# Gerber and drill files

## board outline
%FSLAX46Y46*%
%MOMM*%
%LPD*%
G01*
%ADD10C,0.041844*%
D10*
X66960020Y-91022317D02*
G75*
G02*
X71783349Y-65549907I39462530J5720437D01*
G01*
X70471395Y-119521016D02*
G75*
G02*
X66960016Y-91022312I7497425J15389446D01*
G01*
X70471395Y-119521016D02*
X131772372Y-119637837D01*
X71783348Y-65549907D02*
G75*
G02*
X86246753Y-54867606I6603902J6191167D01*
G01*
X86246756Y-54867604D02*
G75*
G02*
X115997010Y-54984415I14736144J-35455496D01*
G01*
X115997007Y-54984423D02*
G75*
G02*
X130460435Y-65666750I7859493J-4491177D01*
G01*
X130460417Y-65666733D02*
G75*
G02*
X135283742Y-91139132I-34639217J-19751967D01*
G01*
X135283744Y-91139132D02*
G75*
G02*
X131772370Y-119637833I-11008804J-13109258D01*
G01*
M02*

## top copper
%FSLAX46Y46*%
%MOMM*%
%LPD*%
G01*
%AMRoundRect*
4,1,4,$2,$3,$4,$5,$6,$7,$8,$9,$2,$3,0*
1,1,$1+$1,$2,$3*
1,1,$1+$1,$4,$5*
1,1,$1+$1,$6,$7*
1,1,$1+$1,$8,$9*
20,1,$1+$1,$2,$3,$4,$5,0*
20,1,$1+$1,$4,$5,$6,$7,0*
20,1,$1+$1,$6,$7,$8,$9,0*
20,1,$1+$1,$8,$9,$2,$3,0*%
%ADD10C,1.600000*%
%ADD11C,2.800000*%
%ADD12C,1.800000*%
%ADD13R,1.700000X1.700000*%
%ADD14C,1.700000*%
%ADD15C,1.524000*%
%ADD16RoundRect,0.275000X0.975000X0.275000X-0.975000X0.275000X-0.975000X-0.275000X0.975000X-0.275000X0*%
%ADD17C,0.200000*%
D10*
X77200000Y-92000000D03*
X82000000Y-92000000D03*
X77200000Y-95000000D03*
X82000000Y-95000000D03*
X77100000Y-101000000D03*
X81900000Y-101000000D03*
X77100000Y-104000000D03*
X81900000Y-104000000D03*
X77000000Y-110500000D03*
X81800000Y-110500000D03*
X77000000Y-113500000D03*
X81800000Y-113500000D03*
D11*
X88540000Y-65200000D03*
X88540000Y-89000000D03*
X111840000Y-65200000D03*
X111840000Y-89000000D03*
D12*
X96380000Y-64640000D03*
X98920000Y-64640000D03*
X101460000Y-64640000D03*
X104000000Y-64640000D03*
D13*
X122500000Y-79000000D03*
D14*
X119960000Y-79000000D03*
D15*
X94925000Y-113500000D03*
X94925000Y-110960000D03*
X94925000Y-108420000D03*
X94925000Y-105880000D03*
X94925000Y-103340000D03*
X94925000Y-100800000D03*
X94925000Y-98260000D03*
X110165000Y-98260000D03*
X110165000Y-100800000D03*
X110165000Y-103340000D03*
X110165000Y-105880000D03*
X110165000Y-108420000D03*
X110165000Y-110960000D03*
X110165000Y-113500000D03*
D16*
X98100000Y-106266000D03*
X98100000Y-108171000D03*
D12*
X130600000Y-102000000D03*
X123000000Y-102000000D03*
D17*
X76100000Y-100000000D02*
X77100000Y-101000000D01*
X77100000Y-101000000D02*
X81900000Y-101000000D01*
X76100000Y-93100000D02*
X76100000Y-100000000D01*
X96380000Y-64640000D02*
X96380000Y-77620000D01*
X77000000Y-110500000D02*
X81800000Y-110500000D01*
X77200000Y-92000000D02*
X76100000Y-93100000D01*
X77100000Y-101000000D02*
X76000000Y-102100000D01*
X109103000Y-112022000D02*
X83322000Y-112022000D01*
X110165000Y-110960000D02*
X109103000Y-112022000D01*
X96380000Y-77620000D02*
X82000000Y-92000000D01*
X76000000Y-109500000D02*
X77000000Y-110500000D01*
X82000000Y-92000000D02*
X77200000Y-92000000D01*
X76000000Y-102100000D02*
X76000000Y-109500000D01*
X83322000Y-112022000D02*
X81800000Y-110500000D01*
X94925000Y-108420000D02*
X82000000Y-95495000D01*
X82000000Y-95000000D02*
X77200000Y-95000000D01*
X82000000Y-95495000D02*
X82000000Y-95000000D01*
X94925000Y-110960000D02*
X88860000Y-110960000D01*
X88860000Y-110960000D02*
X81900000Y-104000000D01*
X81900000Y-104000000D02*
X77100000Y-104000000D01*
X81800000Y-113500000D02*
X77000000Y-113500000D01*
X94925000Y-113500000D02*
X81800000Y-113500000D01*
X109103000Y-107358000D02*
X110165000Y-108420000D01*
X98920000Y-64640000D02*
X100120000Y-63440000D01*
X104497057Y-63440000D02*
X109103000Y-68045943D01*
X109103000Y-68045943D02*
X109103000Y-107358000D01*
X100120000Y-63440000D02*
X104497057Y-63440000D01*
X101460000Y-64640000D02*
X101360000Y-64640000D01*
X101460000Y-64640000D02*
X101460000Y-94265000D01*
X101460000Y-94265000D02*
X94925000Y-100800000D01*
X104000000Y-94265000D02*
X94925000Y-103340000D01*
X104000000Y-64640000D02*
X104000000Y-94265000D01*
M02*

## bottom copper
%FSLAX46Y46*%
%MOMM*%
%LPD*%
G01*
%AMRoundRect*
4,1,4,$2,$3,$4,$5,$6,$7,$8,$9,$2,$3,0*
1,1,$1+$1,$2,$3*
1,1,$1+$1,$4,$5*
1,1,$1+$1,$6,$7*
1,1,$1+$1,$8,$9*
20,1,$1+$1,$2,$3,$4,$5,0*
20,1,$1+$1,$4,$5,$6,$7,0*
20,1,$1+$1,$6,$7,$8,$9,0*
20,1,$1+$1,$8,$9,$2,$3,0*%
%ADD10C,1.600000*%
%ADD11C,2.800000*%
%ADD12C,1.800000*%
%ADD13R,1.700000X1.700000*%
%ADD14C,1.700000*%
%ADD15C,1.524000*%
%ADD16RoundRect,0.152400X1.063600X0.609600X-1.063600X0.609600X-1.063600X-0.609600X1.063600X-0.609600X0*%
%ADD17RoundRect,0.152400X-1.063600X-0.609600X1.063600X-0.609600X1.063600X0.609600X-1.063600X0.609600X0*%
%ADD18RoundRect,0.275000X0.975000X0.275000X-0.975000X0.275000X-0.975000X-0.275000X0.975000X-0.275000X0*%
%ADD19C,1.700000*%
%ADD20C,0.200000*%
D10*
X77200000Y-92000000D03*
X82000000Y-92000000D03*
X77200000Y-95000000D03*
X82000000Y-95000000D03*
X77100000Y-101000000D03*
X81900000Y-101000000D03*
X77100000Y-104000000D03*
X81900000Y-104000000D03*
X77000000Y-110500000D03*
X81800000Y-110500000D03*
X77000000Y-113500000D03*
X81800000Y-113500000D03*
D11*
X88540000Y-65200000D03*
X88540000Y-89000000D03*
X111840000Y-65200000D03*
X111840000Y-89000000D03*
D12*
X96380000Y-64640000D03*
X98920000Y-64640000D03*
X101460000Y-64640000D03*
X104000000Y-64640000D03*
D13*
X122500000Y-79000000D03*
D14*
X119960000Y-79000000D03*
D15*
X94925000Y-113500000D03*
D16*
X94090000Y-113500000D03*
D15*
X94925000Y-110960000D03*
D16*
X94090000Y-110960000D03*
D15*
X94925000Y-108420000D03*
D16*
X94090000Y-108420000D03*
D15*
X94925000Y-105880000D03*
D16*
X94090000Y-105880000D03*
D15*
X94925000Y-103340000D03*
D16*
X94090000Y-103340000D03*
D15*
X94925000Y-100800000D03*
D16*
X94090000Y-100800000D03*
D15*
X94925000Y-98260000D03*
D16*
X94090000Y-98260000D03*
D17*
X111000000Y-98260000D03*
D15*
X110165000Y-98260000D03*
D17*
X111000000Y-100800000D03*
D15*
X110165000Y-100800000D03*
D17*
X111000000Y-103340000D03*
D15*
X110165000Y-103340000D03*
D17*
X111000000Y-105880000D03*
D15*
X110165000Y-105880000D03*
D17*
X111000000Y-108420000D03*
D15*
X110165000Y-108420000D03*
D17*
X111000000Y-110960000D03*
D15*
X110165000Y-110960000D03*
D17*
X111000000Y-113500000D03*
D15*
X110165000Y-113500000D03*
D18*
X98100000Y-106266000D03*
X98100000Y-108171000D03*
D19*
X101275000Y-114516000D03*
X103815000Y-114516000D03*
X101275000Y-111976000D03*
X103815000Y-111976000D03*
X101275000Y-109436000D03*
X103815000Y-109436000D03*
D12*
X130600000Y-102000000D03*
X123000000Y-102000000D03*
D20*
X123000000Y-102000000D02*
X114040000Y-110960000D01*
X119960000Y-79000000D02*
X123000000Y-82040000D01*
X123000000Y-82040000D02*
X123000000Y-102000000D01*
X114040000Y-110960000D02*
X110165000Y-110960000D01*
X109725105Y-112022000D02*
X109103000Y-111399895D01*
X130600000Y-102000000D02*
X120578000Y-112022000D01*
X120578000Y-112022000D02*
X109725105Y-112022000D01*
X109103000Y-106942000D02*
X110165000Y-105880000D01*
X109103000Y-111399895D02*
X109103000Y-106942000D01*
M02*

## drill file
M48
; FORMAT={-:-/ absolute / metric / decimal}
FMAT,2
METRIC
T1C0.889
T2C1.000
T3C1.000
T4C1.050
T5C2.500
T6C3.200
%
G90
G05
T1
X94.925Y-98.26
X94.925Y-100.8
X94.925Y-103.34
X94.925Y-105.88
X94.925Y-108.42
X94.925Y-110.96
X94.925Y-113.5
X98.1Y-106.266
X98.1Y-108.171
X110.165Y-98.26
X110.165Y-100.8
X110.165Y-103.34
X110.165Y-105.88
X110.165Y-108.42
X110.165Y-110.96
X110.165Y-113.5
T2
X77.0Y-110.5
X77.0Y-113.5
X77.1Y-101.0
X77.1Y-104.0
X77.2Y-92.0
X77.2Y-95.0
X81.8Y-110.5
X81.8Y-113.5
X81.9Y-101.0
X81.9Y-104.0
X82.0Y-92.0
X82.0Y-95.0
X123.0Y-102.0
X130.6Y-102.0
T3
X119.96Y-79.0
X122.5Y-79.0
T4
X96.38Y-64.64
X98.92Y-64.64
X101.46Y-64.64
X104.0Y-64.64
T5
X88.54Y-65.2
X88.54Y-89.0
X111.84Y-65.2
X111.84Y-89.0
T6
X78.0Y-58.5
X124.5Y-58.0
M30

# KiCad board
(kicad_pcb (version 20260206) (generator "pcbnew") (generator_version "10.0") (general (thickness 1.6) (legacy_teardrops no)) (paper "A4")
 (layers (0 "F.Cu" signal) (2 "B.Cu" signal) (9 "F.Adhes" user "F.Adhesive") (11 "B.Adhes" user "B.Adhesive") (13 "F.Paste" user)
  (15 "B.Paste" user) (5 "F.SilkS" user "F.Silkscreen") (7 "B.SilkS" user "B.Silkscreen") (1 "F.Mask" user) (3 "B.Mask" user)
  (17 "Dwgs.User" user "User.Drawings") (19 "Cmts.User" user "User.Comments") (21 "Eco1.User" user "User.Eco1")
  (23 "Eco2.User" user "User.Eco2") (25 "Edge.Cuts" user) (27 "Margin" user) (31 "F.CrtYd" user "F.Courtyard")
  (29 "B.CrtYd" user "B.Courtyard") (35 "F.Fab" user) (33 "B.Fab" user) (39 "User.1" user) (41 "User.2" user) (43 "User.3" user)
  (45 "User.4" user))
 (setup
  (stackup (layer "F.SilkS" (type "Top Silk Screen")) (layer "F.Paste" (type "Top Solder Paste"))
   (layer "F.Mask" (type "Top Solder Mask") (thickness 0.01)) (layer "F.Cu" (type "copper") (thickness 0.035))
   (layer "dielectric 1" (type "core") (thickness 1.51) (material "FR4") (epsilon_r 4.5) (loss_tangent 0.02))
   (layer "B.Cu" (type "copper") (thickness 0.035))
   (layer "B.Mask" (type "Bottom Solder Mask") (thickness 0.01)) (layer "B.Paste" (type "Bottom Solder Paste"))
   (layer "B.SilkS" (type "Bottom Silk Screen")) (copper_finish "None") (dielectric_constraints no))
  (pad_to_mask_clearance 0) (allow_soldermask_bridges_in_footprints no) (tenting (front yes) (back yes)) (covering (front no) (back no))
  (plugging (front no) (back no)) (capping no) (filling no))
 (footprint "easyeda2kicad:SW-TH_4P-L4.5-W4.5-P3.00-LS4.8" (layer "F.Cu") (at 79.6 93.5)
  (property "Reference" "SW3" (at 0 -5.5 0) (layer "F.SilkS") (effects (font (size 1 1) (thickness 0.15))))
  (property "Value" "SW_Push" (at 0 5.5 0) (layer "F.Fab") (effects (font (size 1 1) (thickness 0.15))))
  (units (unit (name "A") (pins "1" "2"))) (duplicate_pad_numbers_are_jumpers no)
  (pad "1" thru_hole circle (at -2.4 -1.5) (size 1.6 1.6) (drill 0.999998) (layers "*.Cu" "*.Mask") (remove_unused_layers no) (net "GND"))
  (pad "1" thru_hole circle (at 2.4 -1.5) (size 1.6 1.6) (drill 0.999998) (layers "*.Cu" "*.Mask") (remove_unused_layers no) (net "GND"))
  (pad "2" thru_hole circle (at -2.4 1.5) (size 1.6 1.6) (drill 0.999998) (layers "*.Cu" "*.Mask") (remove_unused_layers no)
   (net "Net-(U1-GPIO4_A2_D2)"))
  (pad "2" thru_hole circle (at 2.4 1.5) (size 1.6 1.6) (drill 0.999998) (layers "*.Cu" "*.Mask") (remove_unused_layers no)
   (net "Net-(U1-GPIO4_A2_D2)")))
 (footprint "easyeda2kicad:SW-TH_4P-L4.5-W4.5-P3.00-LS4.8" (layer "F.Cu") (at 79.5 102.5)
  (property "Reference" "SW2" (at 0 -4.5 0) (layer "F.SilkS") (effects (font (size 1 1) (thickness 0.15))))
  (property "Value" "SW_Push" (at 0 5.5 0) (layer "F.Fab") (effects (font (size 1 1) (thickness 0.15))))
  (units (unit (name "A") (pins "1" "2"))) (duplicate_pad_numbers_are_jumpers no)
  (pad "1" thru_hole circle (at -2.4 -1.5) (size 1.6 1.6) (drill 0.999998) (layers "*.Cu" "*.Mask") (remove_unused_layers no) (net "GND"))
  (pad "1" thru_hole circle (at 2.4 -1.5) (size 1.6 1.6) (drill 0.999998) (layers "*.Cu" "*.Mask") (remove_unused_layers no) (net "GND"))
  (pad "2" thru_hole circle (at -2.4 1.5) (size 1.6 1.6) (drill 0.999998) (layers "*.Cu" "*.Mask") (remove_unused_layers no)
   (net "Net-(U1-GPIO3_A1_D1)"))
  (pad "2" thru_hole circle (at 2.4 1.5) (size 1.6 1.6) (drill 0.999998) (layers "*.Cu" "*.Mask") (remove_unused_layers no)
   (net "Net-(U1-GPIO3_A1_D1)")))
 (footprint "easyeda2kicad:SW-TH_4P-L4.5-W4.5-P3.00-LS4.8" (layer "F.Cu") (at 79.4 112)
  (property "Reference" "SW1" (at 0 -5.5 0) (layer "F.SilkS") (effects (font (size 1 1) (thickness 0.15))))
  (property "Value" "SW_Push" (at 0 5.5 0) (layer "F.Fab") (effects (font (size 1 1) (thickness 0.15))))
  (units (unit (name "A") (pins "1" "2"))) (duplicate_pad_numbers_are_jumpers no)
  (pad "1" thru_hole circle (at -2.4 -1.5) (size 1.6 1.6) (drill 0.999998) (layers "*.Cu" "*.Mask") (remove_unused_layers no) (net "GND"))
  (pad "1" thru_hole circle (at 2.4 -1.5) (size 1.6 1.6) (drill 0.999998) (layers "*.Cu" "*.Mask") (remove_unused_layers no) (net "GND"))
  (pad "2" thru_hole circle (at -2.4 1.5) (size 1.6 1.6) (drill 0.999998) (layers "*.Cu" "*.Mask") (remove_unused_layers no)
   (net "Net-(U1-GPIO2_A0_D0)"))
  (pad "2" thru_hole circle (at 2.4 1.5) (size 1.6 1.6) (drill 0.999998) (layers "*.Cu" "*.Mask") (remove_unused_layers no)
   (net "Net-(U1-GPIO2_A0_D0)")))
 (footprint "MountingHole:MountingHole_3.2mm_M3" (layer "F.Cu") (at 78 58.5)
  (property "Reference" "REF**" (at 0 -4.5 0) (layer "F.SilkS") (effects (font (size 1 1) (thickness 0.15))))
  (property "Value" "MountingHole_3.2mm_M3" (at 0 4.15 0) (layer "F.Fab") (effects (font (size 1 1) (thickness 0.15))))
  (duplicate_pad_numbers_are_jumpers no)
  (pad "" np_thru_hole circle (at 0 0) (size 3.2 3.2) (drill 3.2) (layers "*.Cu" "*.Mask")))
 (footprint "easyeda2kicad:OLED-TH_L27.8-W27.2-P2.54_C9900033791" (layer "F.Cu") (at 100.19 64.64)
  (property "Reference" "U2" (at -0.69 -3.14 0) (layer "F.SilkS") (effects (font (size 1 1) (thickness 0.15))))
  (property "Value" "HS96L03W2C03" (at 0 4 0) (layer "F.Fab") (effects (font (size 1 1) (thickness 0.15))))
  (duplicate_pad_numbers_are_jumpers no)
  (pad "" thru_hole circle (at -11.65 0.56) (size 2.8 2.8) (drill 2.5) (layers "*.Cu" "*.Mask") (remove_unused_layers no))
  (pad "" thru_hole circle (at -11.65 24.36) (size 2.8 2.8) (drill 2.5) (layers "*.Cu" "*.Mask") (remove_unused_layers no))
  (pad "" thru_hole circle (at 11.65 0.56) (size 2.8 2.8) (drill 2.5) (layers "*.Cu" "*.Mask") (remove_unused_layers no))
  (pad "" thru_hole circle (at 11.65 24.36) (size 2.8 2.8) (drill 2.5) (layers "*.Cu" "*.Mask") (remove_unused_layers no))
  (pad "1" thru_hole circle (at -3.81 0) (size 1.8 1.8) (drill 1.049986) (layers "*.Cu" "*.Mask") (remove_unused_layers no) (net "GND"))
  (pad "2" thru_hole circle (at -1.27 0) (size 1.8 1.8) (drill 1.049986) (layers "*.Cu" "*.Mask") (remove_unused_layers no) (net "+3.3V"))
  (pad "3" thru_hole circle (at 1.27 0) (size 1.8 1.8) (drill 1.049986) (layers "*.Cu" "*.Mask") (remove_unused_layers no)
   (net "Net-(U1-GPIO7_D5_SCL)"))
  (pad "4" thru_hole circle (at 3.81 0) (size 1.8 1.8) (drill 1.049986) (layers "*.Cu" "*.Mask") (remove_unused_layers no)
   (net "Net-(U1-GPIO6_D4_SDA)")))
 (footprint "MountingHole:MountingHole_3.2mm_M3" (layer "F.Cu") (at 124.5 58)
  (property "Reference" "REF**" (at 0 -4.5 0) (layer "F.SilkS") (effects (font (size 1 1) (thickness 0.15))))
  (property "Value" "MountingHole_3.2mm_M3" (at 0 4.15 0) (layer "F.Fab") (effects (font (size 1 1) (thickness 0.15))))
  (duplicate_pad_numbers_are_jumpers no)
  (pad "" np_thru_hole circle (at 0 0) (size 3.2 3.2) (drill 3.2) (layers "*.Cu" "*.Mask")))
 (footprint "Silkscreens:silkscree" (layer "F.Cu") (at 76 75)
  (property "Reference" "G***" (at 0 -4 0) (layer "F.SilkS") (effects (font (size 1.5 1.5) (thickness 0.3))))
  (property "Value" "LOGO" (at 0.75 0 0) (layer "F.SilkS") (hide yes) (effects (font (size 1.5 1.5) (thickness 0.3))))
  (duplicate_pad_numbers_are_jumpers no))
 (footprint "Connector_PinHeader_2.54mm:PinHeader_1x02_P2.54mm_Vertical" (layer "B.Cu") (at 122.5 79 90)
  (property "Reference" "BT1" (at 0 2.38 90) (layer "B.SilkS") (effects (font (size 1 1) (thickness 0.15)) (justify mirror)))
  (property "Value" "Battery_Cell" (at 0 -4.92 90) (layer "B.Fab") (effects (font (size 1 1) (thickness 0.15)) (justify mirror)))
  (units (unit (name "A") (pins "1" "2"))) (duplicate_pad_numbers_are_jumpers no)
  (pad "1" thru_hole rect (at 0 0 90) (size 1.7 1.7) (drill 1) (layers "*.Cu" "*.Mask") (remove_unused_layers no) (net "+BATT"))
  (pad "2" thru_hole circle (at 0 -2.54 90) (size 1.7 1.7) (drill 1) (layers "*.Cu" "*.Mask") (remove_unused_layers no) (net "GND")))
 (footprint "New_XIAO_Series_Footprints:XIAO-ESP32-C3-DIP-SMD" (layer "B.Cu") (at 102.545 105.88 -90)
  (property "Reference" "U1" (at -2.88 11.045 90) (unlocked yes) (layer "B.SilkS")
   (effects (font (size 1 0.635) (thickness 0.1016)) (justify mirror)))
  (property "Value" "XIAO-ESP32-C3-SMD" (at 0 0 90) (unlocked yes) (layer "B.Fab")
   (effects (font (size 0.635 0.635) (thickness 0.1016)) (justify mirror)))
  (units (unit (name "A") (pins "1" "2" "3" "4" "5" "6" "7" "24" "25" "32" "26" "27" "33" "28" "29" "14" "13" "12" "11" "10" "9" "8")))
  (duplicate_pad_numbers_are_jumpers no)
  (pad "1" thru_hole circle (at 7.62 7.62 180) (size 1.524 1.524) (drill 0.889) (layers "*.Cu" "*.Mask") (remove_unused_layers no)
   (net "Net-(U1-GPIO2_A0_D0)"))
  (pad "1" smd roundrect (at 7.62 8.455 180) (size 2.432 1.524) (layers "B.Cu" "B.Mask") (roundrect_rratio 0.1) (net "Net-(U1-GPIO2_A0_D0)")
   (thermal_bridge_angle 45))
  (pad "2" thru_hole circle (at 5.08 7.62 180) (size 1.524 1.524) (drill 0.889) (layers "*.Cu" "*.Mask") (remove_unused_layers no)
   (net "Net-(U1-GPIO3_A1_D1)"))
  (pad "2" smd roundrect (at 5.08 8.455 180) (size 2.432 1.524) (layers "B.Cu" "B.Mask") (roundrect_rratio 0.1) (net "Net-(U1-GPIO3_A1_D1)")
   (thermal_bridge_angle 45))
  (pad "3" thru_hole circle (at 2.54 7.62 180) (size 1.524 1.524) (drill 0.889) (layers "*.Cu" "*.Mask") (remove_unused_layers no)
   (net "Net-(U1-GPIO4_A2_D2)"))
  (pad "3" smd roundrect (at 2.54 8.455 180) (size 2.432 1.524) (layers "B.Cu" "B.Mask") (roundrect_rratio 0.1) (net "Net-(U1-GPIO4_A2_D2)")
   (thermal_bridge_angle 45))
  (pad "4" thru_hole circle (at 0 7.62 180) (size 1.524 1.524) (drill 0.889) (layers "*.Cu" "*.Mask") (remove_unused_layers no)
   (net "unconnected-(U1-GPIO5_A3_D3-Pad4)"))
  (pad "4" smd roundrect (at 0 8.455 180) (size 2.432 1.524) (layers "B.Cu" "B.Mask") (roundrect_rratio 0.1)
   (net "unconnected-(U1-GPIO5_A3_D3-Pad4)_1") (thermal_bridge_angle 45))
  (pad "5" thru_hole circle (at -2.54 7.62 180) (size 1.524 1.524) (drill 0.889) (layers "*.Cu" "*.Mask") (remove_unused_layers no)
   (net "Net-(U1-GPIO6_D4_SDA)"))
  (pad "5" smd roundrect (at -2.54 8.455 180) (size 2.432 1.524) (layers "B.Cu" "B.Mask") (roundrect_rratio 0.1)
   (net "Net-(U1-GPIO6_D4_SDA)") (thermal_bridge_angle 45))
  (pad "6" thru_hole circle (at -5.08 7.62 180) (size 1.524 1.524) (drill 0.889) (layers "*.Cu" "*.Mask") (remove_unused_layers no)
   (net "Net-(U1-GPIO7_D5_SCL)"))
  (pad "6" smd roundrect (at -5.08 8.455 180) (size 2.432 1.524) (layers "B.Cu" "B.Mask") (roundrect_rratio 0.1)
   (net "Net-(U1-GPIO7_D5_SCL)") (thermal_bridge_angle 45))
  (pad "7" thru_hole circle (at -7.62 7.62 180) (size 1.524 1.524) (drill 0.889) (layers "*.Cu" "*.Mask") (remove_unused_layers no)
   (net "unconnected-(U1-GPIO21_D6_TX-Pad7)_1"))
  (pad "7" smd roundrect (at -7.62 8.455 180) (size 2.432 1.524) (layers "B.Cu" "B.Mask") (roundrect_rratio 0.1)
   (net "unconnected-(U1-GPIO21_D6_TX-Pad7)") (thermal_bridge_angle 45))
  (pad "8" smd roundrect (at -7.62 -8.455) (size 2.432 1.524) (layers "B.Cu" "B.Mask") (roundrect_rratio 0.1)
   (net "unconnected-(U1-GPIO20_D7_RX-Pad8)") (thermal_bridge_angle 45))
  (pad "8" thru_hole circle (at -7.62 -7.62) (size 1.524 1.524) (drill 0.889) (layers "*.Cu" "*.Mask") (remove_unused_layers no)
   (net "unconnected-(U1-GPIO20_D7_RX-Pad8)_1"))
  (pad "9" smd roundrect (at -5.08 -8.455) (size 2.432 1.524) (layers "B.Cu" "B.Mask") (roundrect_rratio 0.1)
   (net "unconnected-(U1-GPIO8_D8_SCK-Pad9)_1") (thermal_bridge_angle 45))
  (pad "9" thru_hole circle (at -5.08 -7.62) (size 1.524 1.524) (drill 0.889) (layers "*.Cu" "*.Mask") (remove_unused_layers no)
   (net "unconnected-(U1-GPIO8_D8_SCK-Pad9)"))
  (pad "10" smd roundrect (at -2.54 -8.455) (size 2.432 1.524) (layers "B.Cu" "B.Mask") (roundrect_rratio 0.1)
   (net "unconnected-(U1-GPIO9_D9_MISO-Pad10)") (thermal_bridge_angle 45))
  (pad "10" thru_hole circle (at -2.54 -7.62) (size 1.524 1.524) (drill 0.889) (layers "*.Cu" "*.Mask") (remove_unused_layers no)
   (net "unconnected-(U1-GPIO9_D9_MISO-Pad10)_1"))
  (pad "11" smd roundrect (at 0 -8.455) (size 2.432 1.524) (layers "B.Cu" "B.Mask") (roundrect_rratio 0.1) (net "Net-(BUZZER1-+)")
   (thermal_bridge_angle 45))
  (pad "11" thru_hole circle (at 0 -7.62) (size 1.524 1.524) (drill 0.889) (layers "*.Cu" "*.Mask") (remove_unused_layers no)
   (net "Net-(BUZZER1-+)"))
  (pad "12" smd roundrect (at 2.54 -8.455) (size 2.432 1.524) (layers "B.Cu" "B.Mask") (roundrect_rratio 0.1) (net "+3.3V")
   (thermal_bridge_angle 45))
  (pad "12" thru_hole circle (at 2.54 -7.62) (size 1.524 1.524) (drill 0.889) (layers "*.Cu" "*.Mask") (remove_unused_layers no)
   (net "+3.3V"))
  (pad "13" smd roundrect (at 5.08 -8.455) (size 2.432 1.524) (layers "B.Cu" "B.Mask") (roundrect_rratio 0.1) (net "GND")
   (thermal_bridge_angle 45))
  (pad "13" thru_hole circle (at 5.08 -7.62) (size 1.524 1.524) (drill 0.889) (layers "*.Cu" "*.Mask") (remove_unused_layers no) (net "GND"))
  (pad "14" smd roundrect (at 7.62 -8.455) (size 2.432 1.524) (layers "B.Cu" "B.Mask") (roundrect_rratio 0.1) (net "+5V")
   (thermal_bridge_angle 45))
  (pad "14" thru_hole circle (at 7.62 -7.62) (size 1.524 1.524) (drill 0.889) (layers "*.Cu" "*.Mask") (remove_unused_layers no) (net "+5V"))
  (pad "15" thru_hole roundrect (at 0.386 4.445 180) (size 2.5 1.1) (drill 0.889) (layers "*.Cu" "*.Mask") (remove_unused_layers no)
   (roundrect_rratio 0.25) (thermal_bridge_angle 45))
  (pad "16" thru_hole roundrect (at 2.291 4.445 180) (size 2.5 1.1) (drill 0.889) (layers "*.Cu" "*.Mask") (remove_unused_layers no)
   (roundrect_rratio 0.25) (thermal_bridge_angle 45))
  (pad "17" smd circle (at 8.636 1.27) (size 1.7 1.7) (layers "B.Cu" "B.Mask" "B.Paste"))
  (pad "18" smd circle (at 8.636 -1.27) (size 1.7 1.7) (layers "B.Cu" "B.Mask" "B.Paste"))
  (pad "19" smd circle (at 6.096 1.27) (size 1.7 1.7) (layers "B.Cu" "B.Mask" "B.Paste"))
  (pad "20" smd circle (at 6.096 -1.27) (size 1.7 1.7) (layers "B.Cu" "B.Mask" "B.Paste"))
  (pad "21" smd circle (at 3.556 1.27) (size 1.7 1.7) (layers "B.Cu" "B.Mask" "B.Paste"))
  (pad "22" smd circle (at 3.556 -1.27) (size 1.7 1.7) (layers "B.Cu" "B.Mask" "B.Paste")))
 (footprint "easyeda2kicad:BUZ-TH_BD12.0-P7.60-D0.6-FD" (layer "B.Cu") (at 126.8 102 180)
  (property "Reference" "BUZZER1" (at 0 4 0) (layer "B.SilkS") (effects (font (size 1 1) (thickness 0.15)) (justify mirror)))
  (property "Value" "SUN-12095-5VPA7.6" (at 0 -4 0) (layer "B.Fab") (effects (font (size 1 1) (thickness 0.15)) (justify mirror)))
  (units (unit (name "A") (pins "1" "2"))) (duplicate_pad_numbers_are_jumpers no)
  (pad "1" thru_hole circle (at -3.8 0 180) (size 1.8 1.8) (drill 0.999998) (layers "*.Cu" "*.Mask") (remove_unused_layers no)
   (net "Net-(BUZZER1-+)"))
  (pad "2" thru_hole circle (at 3.8 0 180) (size 1.8 1.8) (drill 0.999998) (layers "*.Cu" "*.Mask") (remove_unused_layers no) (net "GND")))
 (gr_arc (start 66.96002 91.022317) (mid 67.24376 77.883179) (end 71.783348 65.549907) (stroke (width 0.041844) (type default))
  (layer "Edge.Cuts"))
 (gr_arc (start 70.471395 119.521016) (mid 60.978702 106.224956) (end 66.96002 91.022317) (stroke (width 0.041844) (type default))
  (layer "Edge.Cuts"))
 (gr_line (start 70.471395 119.521016) (end 131.772372 119.637837) (stroke (width 0.041844) (type default)) (layer "Edge.Cuts"))
 (gr_arc (start 71.783348 65.549907) (mid 73.009334 52.077252) (end 86.246756 54.867604) (stroke (width 0.041844) (type default))
  (layer "Edge.Cuts"))
 (gr_arc (start 86.246756 54.867604) (mid 101.133655 51.92749) (end 115.997007 54.984423) (stroke (width 0.041844) (type default))
  (layer "Edge.Cuts"))
 (gr_arc (start 115.997007 54.984423) (mid 129.234435 52.194078) (end 130.460417 65.666733) (stroke (width 0.041844) (type default))
  (layer "Edge.Cuts"))
 (gr_arc (start 130.460417 65.666733) (mid 135 78) (end 135.283744 91.139132) (stroke (width 0.041844) (type default)) (layer "Edge.Cuts"))
 (gr_arc (start 135.283744 91.139132) (mid 141.265063 106.341772) (end 131.772372 119.637837) (stroke (width 0.041844) (type default))
  (layer "Edge.Cuts"))
 (segment (start 76.1 100) (end 77.1 101) (width 0.2) (layer "F.Cu") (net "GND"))
 (segment (start 77.1 101) (end 81.9 101) (width 0.2) (layer "F.Cu") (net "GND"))
 (segment (start 76.1 93.1) (end 76.1 100) (width 0.2) (layer "F.Cu") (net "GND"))
 (segment (start 96.38 64.64) (end 96.38 77.62) (width 0.2) (layer "F.Cu") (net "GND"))
 (segment (start 77 110.5) (end 81.8 110.5) (width 0.2) (layer "F.Cu") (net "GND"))
 (segment (start 77.2 92) (end 76.1 93.1) (width 0.2) (layer "F.Cu") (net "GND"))
 (segment (start 77.1 101) (end 76 102.1) (width 0.2) (layer "F.Cu") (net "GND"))
 (segment (start 109.103 112.022) (end 83.322 112.022) (width 0.2) (layer "F.Cu") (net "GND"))
 (segment (start 110.165 110.96) (end 109.103 112.022) (width 0.2) (layer "F.Cu") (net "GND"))
 (segment (start 96.38 77.62) (end 82 92) (width 0.2) (layer "F.Cu") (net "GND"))
 (segment (start 76 109.5) (end 77 110.5) (width 0.2) (layer "F.Cu") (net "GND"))
 (segment (start 82 92) (end 77.2 92) (width 0.2) (layer "F.Cu") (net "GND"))
 (segment (start 76 102.1) (end 76 109.5) (width 0.2) (layer "F.Cu") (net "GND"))
 (segment (start 83.322 112.022) (end 81.8 110.5) (width 0.2) (layer "F.Cu") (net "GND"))
 (segment (start 123 102) (end 114.04 110.96) (width 0.2) (layer "B.Cu") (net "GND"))
 (segment (start 119.96 79) (end 123 82.04) (width 0.2) (layer "B.Cu") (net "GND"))
 (segment (start 123 82.04) (end 123 102) (width 0.2) (layer "B.Cu") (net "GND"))
 (segment (start 114.04 110.96) (end 110.165 110.96) (width 0.2) (layer "B.Cu") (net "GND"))
 (segment (start 94.925 108.42) (end 82 95.495) (width 0.2) (layer "F.Cu") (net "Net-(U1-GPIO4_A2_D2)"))
 (segment (start 82 95) (end 77.2 95) (width 0.2) (layer "F.Cu") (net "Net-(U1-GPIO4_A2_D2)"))
 (segment (start 82 95.495) (end 82 95) (width 0.2) (layer "F.Cu") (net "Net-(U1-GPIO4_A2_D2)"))
 (segment (start 109.725105 112.022) (end 109.103 111.399895) (width 0.2) (layer "B.Cu") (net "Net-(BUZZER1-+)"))
 (segment (start 130.6 102) (end 120.578 112.022) (width 0.2) (layer "B.Cu") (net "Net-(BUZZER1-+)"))
 (segment (start 120.578 112.022) (end 109.725105 112.022) (width 0.2) (layer "B.Cu") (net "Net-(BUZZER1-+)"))
 (segment (start 109.103 106.942) (end 110.165 105.88) (width 0.2) (layer "B.Cu") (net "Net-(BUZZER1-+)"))
 (segment (start 109.103 111.399895) (end 109.103 106.942) (width 0.2) (layer "B.Cu") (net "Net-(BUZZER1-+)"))
 (segment (start 94.925 110.96) (end 88.86 110.96) (width 0.2) (layer "F.Cu") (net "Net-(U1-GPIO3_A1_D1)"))
 (segment (start 88.86 110.96) (end 81.9 104) (width 0.2) (layer "F.Cu") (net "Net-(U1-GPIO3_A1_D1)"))
 (segment (start 81.9 104) (end 77.1 104) (width 0.2) (layer "F.Cu") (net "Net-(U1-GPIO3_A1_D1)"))
 (segment (start 81.8 113.5) (end 77 113.5) (width 0.2) (layer "F.Cu") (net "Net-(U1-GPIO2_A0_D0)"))
 (segment (start 94.925 113.5) (end 81.8 113.5) (width 0.2) (layer "F.Cu") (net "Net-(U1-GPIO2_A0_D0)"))
 (segment (start 109.103 107.358) (end 110.165 108.42) (width 0.2) (layer "F.Cu") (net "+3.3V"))
 (segment (start 98.92 64.64) (end 100.12 63.44) (width 0.2) (layer "F.Cu") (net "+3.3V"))
 (segment (start 104.497057 63.44) (end 109.103 68.045943) (width 0.2) (layer "F.Cu") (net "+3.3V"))
 (segment (start 109.103 68.045943) (end 109.103 107.358) (width 0.2) (layer "F.Cu") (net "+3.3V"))
 (segment (start 100.12 63.44) (end 104.497057 63.44) (width 0.2) (layer "F.Cu") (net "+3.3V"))
 (segment (start 101.46 64.64) (end 101.36 64.64) (width 0.2) (layer "F.Cu") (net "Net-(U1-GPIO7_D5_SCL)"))
 (segment (start 101.46 64.64) (end 101.46 94.265) (width 0.2) (layer "F.Cu") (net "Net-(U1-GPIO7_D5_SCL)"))
 (segment (start 101.46 94.265) (end 94.925 100.8) (width 0.2) (layer "F.Cu") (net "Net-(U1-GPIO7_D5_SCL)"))
 (segment (start 104 94.265) (end 94.925 103.34) (width 0.2) (layer "F.Cu") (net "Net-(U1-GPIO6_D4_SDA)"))
 (segment (start 104 64.64) (end 104 94.265) (width 0.2) (layer "F.Cu") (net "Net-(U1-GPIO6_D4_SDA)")))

